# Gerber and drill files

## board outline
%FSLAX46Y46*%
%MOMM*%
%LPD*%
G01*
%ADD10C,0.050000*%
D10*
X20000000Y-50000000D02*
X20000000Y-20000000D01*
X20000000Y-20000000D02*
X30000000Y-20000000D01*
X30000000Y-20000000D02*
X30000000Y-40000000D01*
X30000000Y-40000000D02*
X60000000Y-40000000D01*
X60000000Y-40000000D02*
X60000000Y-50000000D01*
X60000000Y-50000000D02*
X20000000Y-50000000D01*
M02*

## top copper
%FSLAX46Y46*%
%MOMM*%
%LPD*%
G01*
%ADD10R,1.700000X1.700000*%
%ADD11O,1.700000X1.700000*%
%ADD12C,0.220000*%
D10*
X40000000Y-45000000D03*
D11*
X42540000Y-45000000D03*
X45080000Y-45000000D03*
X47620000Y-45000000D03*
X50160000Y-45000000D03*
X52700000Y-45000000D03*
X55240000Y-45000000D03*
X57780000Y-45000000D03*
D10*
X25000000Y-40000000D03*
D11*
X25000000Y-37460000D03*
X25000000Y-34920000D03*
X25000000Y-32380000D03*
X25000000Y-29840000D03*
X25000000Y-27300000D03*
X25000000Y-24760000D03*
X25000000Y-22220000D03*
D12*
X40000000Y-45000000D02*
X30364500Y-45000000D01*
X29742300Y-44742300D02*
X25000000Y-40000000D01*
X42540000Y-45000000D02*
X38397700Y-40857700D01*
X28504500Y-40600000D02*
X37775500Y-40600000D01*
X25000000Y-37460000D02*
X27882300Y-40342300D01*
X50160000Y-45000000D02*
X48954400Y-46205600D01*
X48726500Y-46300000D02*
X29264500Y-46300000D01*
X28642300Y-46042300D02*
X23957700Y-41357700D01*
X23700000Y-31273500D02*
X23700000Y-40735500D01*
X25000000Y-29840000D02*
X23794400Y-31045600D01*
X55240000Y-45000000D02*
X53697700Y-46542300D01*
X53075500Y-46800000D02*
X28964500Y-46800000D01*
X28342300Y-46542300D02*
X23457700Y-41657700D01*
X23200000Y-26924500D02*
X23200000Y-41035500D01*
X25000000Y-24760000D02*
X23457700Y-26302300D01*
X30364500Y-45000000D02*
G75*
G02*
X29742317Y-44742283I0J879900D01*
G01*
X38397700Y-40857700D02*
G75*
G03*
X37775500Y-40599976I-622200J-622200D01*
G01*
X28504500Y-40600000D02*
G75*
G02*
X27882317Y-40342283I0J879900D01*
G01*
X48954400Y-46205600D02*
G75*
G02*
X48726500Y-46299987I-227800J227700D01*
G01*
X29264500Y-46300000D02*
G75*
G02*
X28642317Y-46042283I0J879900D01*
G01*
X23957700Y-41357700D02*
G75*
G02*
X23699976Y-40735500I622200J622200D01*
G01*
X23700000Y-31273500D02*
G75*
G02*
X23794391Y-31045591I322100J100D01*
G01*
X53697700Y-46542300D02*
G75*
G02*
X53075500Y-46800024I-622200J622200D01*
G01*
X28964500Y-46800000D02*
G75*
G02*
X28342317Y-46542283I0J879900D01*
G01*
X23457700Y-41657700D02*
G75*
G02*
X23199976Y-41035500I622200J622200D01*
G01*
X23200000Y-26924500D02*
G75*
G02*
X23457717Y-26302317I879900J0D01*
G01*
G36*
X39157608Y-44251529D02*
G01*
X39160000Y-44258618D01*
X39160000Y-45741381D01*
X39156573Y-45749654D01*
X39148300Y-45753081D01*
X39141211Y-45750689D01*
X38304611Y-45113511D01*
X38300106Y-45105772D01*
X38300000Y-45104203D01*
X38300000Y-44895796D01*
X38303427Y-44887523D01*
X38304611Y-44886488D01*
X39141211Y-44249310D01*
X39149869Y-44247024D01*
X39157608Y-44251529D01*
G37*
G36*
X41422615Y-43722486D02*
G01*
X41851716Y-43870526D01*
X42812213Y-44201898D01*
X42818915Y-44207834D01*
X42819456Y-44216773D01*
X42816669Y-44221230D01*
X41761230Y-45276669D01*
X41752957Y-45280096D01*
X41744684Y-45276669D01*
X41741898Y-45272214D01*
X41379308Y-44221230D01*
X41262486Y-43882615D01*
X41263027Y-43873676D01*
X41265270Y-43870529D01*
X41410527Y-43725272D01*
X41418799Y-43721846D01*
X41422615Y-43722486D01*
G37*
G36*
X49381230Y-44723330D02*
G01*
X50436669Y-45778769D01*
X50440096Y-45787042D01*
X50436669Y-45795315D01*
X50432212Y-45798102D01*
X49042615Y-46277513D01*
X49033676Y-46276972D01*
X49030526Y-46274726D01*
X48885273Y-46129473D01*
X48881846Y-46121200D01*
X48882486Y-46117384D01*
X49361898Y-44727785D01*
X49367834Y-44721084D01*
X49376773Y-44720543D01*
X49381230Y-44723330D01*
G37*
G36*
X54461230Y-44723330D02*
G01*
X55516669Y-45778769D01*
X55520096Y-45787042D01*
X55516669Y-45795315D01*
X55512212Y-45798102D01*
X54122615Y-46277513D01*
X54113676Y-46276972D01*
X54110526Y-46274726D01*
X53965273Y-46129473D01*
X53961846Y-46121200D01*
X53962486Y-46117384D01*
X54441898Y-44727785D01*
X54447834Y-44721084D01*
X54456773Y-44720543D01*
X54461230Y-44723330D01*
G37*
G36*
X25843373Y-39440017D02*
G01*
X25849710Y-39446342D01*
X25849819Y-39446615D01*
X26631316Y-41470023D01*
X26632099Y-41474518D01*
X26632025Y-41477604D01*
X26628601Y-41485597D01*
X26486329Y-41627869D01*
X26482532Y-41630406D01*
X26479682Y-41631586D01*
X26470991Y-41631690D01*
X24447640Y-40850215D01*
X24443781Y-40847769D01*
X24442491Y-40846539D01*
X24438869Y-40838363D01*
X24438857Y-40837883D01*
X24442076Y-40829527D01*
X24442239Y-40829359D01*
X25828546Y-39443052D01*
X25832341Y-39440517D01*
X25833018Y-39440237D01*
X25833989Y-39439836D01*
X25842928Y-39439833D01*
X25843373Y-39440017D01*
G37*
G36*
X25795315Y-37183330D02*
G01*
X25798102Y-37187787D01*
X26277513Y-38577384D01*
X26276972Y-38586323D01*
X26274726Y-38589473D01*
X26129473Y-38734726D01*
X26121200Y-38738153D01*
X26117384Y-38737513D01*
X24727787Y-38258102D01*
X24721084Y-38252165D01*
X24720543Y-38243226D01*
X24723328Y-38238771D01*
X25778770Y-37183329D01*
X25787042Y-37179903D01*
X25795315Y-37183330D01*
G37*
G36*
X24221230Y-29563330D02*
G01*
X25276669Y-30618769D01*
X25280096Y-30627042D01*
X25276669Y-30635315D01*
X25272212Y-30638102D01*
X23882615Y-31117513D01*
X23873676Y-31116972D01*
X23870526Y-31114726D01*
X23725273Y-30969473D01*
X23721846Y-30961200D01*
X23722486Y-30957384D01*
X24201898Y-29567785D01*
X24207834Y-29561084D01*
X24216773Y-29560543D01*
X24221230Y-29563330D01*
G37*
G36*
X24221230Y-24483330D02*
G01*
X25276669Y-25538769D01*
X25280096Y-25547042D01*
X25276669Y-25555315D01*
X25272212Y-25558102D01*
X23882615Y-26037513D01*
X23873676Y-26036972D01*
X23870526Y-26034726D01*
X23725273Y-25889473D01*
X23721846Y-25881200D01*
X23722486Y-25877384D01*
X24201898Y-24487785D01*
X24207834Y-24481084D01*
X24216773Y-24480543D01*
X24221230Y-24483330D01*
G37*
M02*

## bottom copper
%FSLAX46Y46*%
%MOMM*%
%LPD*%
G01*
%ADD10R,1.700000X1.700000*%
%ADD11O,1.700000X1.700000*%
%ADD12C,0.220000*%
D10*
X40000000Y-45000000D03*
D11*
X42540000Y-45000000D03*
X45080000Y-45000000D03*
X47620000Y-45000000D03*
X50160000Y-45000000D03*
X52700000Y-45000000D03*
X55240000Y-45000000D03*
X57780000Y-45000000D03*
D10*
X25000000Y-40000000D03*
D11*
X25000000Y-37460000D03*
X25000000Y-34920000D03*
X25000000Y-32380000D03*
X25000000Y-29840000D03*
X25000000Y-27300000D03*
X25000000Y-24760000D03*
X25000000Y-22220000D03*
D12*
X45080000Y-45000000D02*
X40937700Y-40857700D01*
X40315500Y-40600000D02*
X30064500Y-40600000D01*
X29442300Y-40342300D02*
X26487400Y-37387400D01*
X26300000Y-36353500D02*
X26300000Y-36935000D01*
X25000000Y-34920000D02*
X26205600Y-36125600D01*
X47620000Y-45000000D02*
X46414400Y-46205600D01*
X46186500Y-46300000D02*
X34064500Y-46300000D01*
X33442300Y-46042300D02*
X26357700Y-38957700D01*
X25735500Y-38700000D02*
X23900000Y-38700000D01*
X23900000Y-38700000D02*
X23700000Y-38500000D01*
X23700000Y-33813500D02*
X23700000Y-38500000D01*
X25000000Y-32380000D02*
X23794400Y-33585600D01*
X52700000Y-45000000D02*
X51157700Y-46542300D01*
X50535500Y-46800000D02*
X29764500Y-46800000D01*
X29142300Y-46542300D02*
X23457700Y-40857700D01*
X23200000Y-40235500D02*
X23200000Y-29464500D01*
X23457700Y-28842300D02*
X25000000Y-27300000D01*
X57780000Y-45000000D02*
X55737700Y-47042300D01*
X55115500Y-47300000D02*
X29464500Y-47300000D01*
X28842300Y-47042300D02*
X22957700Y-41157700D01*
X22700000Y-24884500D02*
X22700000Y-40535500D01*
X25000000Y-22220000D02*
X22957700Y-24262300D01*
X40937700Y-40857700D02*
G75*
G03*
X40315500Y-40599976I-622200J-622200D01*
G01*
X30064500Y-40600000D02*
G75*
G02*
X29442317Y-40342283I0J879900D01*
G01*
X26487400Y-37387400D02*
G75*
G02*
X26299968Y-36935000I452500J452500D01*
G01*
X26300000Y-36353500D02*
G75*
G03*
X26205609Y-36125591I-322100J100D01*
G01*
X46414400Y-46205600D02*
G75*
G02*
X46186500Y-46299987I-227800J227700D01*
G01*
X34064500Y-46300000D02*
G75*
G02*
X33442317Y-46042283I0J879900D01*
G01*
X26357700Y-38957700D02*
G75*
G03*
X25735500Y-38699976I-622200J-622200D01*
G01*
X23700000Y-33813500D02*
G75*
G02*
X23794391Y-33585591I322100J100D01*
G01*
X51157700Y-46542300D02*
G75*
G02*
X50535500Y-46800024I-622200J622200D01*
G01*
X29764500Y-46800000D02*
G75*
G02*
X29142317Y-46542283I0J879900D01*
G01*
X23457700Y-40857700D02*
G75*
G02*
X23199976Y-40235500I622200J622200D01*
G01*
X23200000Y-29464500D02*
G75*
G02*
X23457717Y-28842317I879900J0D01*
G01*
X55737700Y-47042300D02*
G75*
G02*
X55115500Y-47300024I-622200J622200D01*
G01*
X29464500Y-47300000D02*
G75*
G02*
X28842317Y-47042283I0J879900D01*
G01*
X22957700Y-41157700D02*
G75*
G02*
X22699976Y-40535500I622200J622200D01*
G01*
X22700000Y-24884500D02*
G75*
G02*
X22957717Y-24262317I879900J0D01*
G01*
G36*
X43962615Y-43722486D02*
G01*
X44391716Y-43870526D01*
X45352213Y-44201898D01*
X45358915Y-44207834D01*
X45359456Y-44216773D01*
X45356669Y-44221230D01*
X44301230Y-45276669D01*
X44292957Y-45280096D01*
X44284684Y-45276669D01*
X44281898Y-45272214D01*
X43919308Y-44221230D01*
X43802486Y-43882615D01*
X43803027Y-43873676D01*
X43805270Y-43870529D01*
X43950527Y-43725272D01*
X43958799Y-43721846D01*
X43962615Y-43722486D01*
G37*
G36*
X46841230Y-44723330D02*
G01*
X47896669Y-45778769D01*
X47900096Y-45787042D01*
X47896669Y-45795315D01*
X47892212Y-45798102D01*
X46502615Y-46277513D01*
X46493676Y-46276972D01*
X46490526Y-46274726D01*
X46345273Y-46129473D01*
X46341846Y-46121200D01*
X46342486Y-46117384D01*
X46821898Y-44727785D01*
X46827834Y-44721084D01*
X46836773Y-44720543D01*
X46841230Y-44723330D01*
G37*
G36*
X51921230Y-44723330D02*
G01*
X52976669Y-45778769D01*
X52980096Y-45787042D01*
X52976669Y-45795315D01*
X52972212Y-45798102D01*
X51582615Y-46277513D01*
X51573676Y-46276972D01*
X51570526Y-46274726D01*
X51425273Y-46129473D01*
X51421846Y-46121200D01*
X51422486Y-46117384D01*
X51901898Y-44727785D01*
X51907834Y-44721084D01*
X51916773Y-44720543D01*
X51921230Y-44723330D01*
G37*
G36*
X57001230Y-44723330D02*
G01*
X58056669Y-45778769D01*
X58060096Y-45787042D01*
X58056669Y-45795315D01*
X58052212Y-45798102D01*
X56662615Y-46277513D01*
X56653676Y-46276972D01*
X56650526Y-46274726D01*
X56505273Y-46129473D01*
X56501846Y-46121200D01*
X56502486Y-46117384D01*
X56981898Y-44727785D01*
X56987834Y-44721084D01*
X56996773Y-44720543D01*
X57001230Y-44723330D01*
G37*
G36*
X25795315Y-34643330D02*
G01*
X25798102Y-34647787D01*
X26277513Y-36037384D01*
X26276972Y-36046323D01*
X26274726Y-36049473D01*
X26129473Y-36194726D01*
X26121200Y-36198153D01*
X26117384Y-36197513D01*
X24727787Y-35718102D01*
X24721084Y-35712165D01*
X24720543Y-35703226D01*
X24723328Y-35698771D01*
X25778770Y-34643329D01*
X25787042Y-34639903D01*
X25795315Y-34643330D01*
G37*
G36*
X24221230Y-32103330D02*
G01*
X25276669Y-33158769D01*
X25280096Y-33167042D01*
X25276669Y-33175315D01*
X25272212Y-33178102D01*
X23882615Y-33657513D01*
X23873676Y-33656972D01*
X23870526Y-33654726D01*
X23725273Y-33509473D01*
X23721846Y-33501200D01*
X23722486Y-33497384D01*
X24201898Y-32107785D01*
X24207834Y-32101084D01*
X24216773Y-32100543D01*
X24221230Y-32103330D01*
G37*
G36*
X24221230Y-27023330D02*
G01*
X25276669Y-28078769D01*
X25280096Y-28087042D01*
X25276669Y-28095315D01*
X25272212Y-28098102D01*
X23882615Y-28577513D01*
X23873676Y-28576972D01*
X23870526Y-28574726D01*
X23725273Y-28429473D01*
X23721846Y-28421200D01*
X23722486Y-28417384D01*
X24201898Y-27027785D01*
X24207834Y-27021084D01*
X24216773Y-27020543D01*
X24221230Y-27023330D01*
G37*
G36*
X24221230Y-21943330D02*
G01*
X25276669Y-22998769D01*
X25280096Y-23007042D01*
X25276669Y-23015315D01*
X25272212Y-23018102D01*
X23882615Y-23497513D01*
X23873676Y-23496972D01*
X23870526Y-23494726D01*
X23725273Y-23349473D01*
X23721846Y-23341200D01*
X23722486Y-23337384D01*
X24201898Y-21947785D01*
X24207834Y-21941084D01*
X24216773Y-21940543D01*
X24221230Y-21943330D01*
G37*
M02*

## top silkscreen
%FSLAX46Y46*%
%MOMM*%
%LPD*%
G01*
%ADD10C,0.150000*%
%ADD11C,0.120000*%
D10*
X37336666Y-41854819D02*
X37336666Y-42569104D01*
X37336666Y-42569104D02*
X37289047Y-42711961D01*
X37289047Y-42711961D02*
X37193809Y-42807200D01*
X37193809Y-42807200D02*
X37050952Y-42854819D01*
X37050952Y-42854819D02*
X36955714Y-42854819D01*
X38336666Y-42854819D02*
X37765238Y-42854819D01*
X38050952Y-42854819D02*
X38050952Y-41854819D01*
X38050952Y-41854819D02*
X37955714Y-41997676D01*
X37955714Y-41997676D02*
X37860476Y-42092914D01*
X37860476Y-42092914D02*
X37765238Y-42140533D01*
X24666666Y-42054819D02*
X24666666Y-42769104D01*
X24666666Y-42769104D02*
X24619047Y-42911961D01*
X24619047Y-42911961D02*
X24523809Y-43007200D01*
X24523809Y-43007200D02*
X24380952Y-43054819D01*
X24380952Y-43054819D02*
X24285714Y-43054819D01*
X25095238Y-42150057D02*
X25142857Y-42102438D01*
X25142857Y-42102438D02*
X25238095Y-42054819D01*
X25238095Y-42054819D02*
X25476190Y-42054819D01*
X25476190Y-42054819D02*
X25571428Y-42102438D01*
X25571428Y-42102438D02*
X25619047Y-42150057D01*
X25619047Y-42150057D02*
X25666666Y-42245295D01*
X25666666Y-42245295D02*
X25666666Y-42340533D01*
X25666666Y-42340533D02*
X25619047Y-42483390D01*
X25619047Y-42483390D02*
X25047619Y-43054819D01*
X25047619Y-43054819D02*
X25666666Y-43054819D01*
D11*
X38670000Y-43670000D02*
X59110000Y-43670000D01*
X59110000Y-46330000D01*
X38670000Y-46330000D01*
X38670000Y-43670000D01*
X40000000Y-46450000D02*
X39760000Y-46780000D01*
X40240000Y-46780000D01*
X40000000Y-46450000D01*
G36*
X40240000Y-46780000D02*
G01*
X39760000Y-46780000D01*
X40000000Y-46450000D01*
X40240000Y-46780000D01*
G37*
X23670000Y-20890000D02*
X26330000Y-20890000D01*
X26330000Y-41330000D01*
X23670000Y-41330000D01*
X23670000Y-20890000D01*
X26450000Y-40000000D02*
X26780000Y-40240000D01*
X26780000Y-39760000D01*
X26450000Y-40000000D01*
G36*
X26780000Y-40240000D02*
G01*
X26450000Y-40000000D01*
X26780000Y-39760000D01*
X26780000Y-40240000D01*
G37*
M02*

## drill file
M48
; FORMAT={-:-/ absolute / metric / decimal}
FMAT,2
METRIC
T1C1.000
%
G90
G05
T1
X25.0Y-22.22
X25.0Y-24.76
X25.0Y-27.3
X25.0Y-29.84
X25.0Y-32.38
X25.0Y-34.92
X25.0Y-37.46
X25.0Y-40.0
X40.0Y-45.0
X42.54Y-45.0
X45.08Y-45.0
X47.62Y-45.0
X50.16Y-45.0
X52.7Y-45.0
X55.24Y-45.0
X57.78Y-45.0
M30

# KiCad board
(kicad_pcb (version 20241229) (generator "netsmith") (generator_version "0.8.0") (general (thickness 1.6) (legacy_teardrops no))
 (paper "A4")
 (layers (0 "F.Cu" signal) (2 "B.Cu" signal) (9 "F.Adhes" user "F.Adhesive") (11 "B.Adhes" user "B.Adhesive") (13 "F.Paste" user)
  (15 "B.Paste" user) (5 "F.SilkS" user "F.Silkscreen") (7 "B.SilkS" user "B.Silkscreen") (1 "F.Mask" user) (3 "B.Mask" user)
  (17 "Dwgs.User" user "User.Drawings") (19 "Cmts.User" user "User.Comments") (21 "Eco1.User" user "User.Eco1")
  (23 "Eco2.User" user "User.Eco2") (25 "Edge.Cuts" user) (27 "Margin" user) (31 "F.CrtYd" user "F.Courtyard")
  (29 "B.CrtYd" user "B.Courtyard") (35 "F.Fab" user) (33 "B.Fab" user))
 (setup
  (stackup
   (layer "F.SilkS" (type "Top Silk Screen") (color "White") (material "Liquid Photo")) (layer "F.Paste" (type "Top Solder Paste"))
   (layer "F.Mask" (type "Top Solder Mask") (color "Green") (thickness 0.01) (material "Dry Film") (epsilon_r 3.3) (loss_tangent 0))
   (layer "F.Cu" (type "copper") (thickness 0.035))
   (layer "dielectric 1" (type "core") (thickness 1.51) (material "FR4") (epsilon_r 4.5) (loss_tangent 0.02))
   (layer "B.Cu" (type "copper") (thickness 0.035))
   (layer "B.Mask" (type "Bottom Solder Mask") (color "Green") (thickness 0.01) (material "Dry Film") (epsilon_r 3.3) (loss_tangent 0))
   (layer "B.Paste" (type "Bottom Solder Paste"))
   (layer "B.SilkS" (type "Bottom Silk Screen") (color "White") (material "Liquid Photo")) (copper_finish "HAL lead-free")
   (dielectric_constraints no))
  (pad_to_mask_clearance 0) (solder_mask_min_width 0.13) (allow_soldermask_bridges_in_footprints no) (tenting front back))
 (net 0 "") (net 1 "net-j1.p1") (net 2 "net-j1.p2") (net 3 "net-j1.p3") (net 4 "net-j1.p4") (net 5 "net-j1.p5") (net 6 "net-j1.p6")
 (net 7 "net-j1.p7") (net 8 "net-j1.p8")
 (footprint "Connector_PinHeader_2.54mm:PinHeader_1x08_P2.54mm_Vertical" (layer "F.Cu") (at 40 45 90)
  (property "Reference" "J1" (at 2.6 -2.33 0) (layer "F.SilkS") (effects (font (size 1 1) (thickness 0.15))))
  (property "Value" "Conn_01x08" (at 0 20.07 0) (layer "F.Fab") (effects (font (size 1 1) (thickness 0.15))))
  (pad "1" thru_hole rect (at 0 0 90) (size 1.7 1.7) (drill 1) (layers "*.Cu" "*.Mask") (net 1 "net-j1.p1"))
  (pad "2" thru_hole oval (at 0 2.54 90) (size 1.7 1.7) (drill 1) (layers "*.Cu" "*.Mask") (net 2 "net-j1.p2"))
  (pad "3" thru_hole oval (at 0 5.08 90) (size 1.7 1.7) (drill 1) (layers "*.Cu" "*.Mask") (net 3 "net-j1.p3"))
  (pad "4" thru_hole oval (at 0 7.62 90) (size 1.7 1.7) (drill 1) (layers "*.Cu" "*.Mask") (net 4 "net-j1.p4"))
  (pad "5" thru_hole oval (at 0 10.16 90) (size 1.7 1.7) (drill 1) (layers "*.Cu" "*.Mask") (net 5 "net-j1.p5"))
  (pad "6" thru_hole oval (at 0 12.7 90) (size 1.7 1.7) (drill 1) (layers "*.Cu" "*.Mask") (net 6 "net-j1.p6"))
  (pad "7" thru_hole oval (at 0 15.24 90) (size 1.7 1.7) (drill 1) (layers "*.Cu" "*.Mask") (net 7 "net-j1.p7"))
  (pad "8" thru_hole oval (at 0 17.78 90) (size 1.7 1.7) (drill 1) (layers "*.Cu" "*.Mask") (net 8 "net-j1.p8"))
  (fp_rect (start -1.33 -1.33) (end 1.33 19.11) (stroke (width 0.12) (type solid)) (fill no) (layer "F.SilkS"))
  (fp_poly (pts (xy -1.45 0) (xy -1.78 -0.24) (xy -1.78 0.24)) (stroke (width 0.12) (type solid)) (fill solid) (layer "F.SilkS")))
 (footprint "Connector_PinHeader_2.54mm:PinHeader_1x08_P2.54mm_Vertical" (layer "F.Cu") (at 25 40 180)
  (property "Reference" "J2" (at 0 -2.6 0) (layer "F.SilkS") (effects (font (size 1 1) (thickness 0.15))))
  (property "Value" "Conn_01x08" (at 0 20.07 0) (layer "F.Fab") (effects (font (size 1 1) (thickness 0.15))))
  (pad "1" thru_hole rect (at 0 0 180) (size 1.7 1.7) (drill 1) (layers "*.Cu" "*.Mask") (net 1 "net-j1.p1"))
  (pad "2" thru_hole oval (at 0 2.54 180) (size 1.7 1.7) (drill 1) (layers "*.Cu" "*.Mask") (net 2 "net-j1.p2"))
  (pad "3" thru_hole oval (at 0 5.08 180) (size 1.7 1.7) (drill 1) (layers "*.Cu" "*.Mask") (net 3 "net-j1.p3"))
  (pad "4" thru_hole oval (at 0 7.62 180) (size 1.7 1.7) (drill 1) (layers "*.Cu" "*.Mask") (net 4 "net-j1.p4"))
  (pad "5" thru_hole oval (at 0 10.16 180) (size 1.7 1.7) (drill 1) (layers "*.Cu" "*.Mask") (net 5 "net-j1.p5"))
  (pad "6" thru_hole oval (at 0 12.7 180) (size 1.7 1.7) (drill 1) (layers "*.Cu" "*.Mask") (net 6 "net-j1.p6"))
  (pad "7" thru_hole oval (at 0 15.24 180) (size 1.7 1.7) (drill 1) (layers "*.Cu" "*.Mask") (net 7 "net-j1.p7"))
  (pad "8" thru_hole oval (at 0 17.78 180) (size 1.7 1.7) (drill 1) (layers "*.Cu" "*.Mask") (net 8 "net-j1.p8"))
  (fp_rect (start -1.33 -1.33) (end 1.33 19.11) (stroke (width 0.12) (type solid)) (fill no) (layer "F.SilkS"))
  (fp_poly (pts (xy -1.45 0) (xy -1.78 -0.24) (xy -1.78 0.24)) (stroke (width 0.12) (type solid)) (fill solid) (layer "F.SilkS")))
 (segment (start 40 45) (end 30.3645 45) (width 0.22) (layer "F.Cu") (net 1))
 (segment (start 29.7423 44.7423) (end 25 40) (width 0.22) (layer "F.Cu") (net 1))
 (segment (start 42.54 45) (end 38.3977 40.8577) (width 0.22) (layer "F.Cu") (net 2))
 (segment (start 28.5045 40.6) (end 37.7755 40.6) (width 0.22) (layer "F.Cu") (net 2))
 (segment (start 25 37.46) (end 27.8823 40.3423) (width 0.22) (layer "F.Cu") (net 2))
 (segment (start 45.08 45) (end 40.9377 40.8577) (width 0.22) (layer "B.Cu") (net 3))
 (segment (start 40.3155 40.6) (end 30.0645 40.6) (width 0.22) (layer "B.Cu") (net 3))
 (segment (start 29.4423 40.3423) (end 26.4874 37.3874) (width 0.22) (layer "B.Cu") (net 3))
 (segment (start 26.3 36.3535) (end 26.3 36.935) (width 0.22) (layer "B.Cu") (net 3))
 (segment (start 25 34.92) (end 26.2056 36.1256) (width 0.22) (layer "B.Cu") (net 3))
 (segment (start 47.62 45) (end 46.4144 46.2056) (width 0.22) (layer "B.Cu") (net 4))
 (segment (start 46.1865 46.3) (end 34.0645 46.3) (width 0.22) (layer "B.Cu") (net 4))
 (segment (start 33.4423 46.0423) (end 26.3577 38.9577) (width 0.22) (layer "B.Cu") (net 4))
 (segment (start 25.7355 38.7) (end 23.9 38.7) (width 0.22) (layer "B.Cu") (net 4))
 (segment (start 23.9 38.7) (end 23.7 38.5) (width 0.22) (layer "B.Cu") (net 4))
 (segment (start 23.7 33.8135) (end 23.7 38.5) (width 0.22) (layer "B.Cu") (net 4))
 (segment (start 25 32.38) (end 23.7944 33.5856) (width 0.22) (layer "B.Cu") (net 4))
 (segment (start 50.16 45) (end 48.9544 46.2056) (width 0.22) (layer "F.Cu") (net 5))
 (segment (start 48.7265 46.3) (end 29.2645 46.3) (width 0.22) (layer "F.Cu") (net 5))
 (segment (start 28.6423 46.0423) (end 23.9577 41.3577) (width 0.22) (layer "F.Cu") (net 5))
 (segment (start 23.7 31.2735) (end 23.7 40.7355) (width 0.22) (layer "F.Cu") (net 5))
 (segment (start 25 29.84) (end 23.7944 31.0456) (width 0.22) (layer "F.Cu") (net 5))
 (segment (start 52.7 45) (end 51.1577 46.5423) (width 0.22) (layer "B.Cu") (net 6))
 (segment (start 50.5355 46.8) (end 29.7645 46.8) (width 0.22) (layer "B.Cu") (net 6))
 (segment (start 29.1423 46.5423) (end 23.4577 40.8577) (width 0.22) (layer "B.Cu") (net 6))
 (segment (start 23.2 40.2355) (end 23.2 29.4645) (width 0.22) (layer "B.Cu") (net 6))
 (segment (start 23.4577 28.8423) (end 25 27.3) (width 0.22) (layer "B.Cu") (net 6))
 (segment (start 55.24 45) (end 53.6977 46.5423) (width 0.22) (layer "F.Cu") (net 7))
 (segment (start 53.0755 46.8) (end 28.9645 46.8) (width 0.22) (layer "F.Cu") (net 7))
 (segment (start 28.3423 46.5423) (end 23.4577 41.6577) (width 0.22) (layer "F.Cu") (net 7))
 (segment (start 23.2 26.9245) (end 23.2 41.0355) (width 0.22) (layer "F.Cu") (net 7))
 (segment (start 25 24.76) (end 23.4577 26.3023) (width 0.22) (layer "F.Cu") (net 7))
 (segment (start 57.78 45) (end 55.7377 47.0423) (width 0.22) (layer "B.Cu") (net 8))
 (segment (start 55.1155 47.3) (end 29.4645 47.3) (width 0.22) (layer "B.Cu") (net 8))
 (segment (start 28.8423 47.0423) (end 22.9577 41.1577) (width 0.22) (layer "B.Cu") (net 8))
 (segment (start 22.7 24.8845) (end 22.7 40.5355) (width 0.22) (layer "B.Cu") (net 8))
 (segment (start 25 22.22) (end 22.9577 24.2623) (width 0.22) (layer "B.Cu") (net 8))
 (arc (start 30.3645 45) (mid 30.0277 44.933) (end 29.7423 44.7423) (width 0.22) (layer "F.Cu") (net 1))
 (arc (start 38.3977 40.8577) (mid 38.1123 40.667) (end 37.7755 40.6) (width 0.22) (layer "F.Cu") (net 2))
 (arc (start 28.5045 40.6) (mid 28.1677 40.533) (end 27.8823 40.3423) (width 0.22) (layer "F.Cu") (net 2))
 (arc (start 40.9377 40.8577) (mid 40.6523 40.667) (end 40.3155 40.6) (width 0.22) (layer "B.Cu") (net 3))
 (arc (start 30.0645 40.6) (mid 29.7277 40.533) (end 29.4423 40.3423) (width 0.22) (layer "B.Cu") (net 3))
 (arc (start 26.4874 37.3874) (mid 26.3487 37.1798) (end 26.3 36.935) (width 0.22) (layer "B.Cu") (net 3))
 (arc (start 26.3 36.3535) (mid 26.2755 36.2302) (end 26.2056 36.1256) (width 0.22) (layer "B.Cu") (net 3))
 (arc (start 46.4144 46.2056) (mid 46.3098 46.2755) (end 46.1865 46.3) (width 0.22) (layer "B.Cu") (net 4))
 (arc (start 34.0645 46.3) (mid 33.7277 46.233) (end 33.4423 46.0423) (width 0.22) (layer "B.Cu") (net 4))
 (arc (start 26.3577 38.9577) (mid 26.0723 38.767) (end 25.7355 38.7) (width 0.22) (layer "B.Cu") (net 4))
 (arc (start 23.7 33.8135) (mid 23.7245 33.6902) (end 23.7944 33.5856) (width 0.22) (layer "B.Cu") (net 4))
 (arc (start 48.9544 46.2056) (mid 48.8498 46.2755) (end 48.7265 46.3) (width 0.22) (layer "F.Cu") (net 5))
 (arc (start 29.2645 46.3) (mid 28.9277 46.233) (end 28.6423 46.0423) (width 0.22) (layer "F.Cu") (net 5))
 (arc (start 23.9577 41.3577) (mid 23.767 41.0723) (end 23.7 40.7355) (width 0.22) (layer "F.Cu") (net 5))
 (arc (start 23.7 31.2735) (mid 23.7245 31.1502) (end 23.7944 31.0456) (width 0.22) (layer "F.Cu") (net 5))
 (arc (start 51.1577 46.5423) (mid 50.8723 46.733) (end 50.5355 46.8) (width 0.22) (layer "B.Cu") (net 6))
 (arc (start 29.7645 46.8) (mid 29.4277 46.733) (end 29.1423 46.5423) (width 0.22) (layer "B.Cu") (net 6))
 (arc (start 23.4577 40.8577) (mid 23.267 40.5723) (end 23.2 40.2355) (width 0.22) (layer "B.Cu") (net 6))
 (arc (start 23.2 29.4645) (mid 23.267 29.1277) (end 23.4577 28.8423) (width 0.22) (layer "B.Cu") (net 6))
 (arc (start 53.6977 46.5423) (mid 53.4123 46.733) (end 53.0755 46.8) (width 0.22) (layer "F.Cu") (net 7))
 (arc (start 28.9645 46.8) (mid 28.6277 46.733) (end 28.3423 46.5423) (width 0.22) (layer "F.Cu") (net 7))
 (arc (start 23.4577 41.6577) (mid 23.267 41.3723) (end 23.2 41.0355) (width 0.22) (layer "F.Cu") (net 7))
 (arc (start 23.2 26.9245) (mid 23.267 26.5877) (end 23.4577 26.3023) (width 0.22) (layer "F.Cu") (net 7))
 (arc (start 55.7377 47.0423) (mid 55.4523 47.233) (end 55.1155 47.3) (width 0.22) (layer "B.Cu") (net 8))
 (arc (start 29.4645 47.3) (mid 29.1277 47.233) (end 28.8423 47.0423) (width 0.22) (layer "B.Cu") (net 8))
 (arc (start 22.9577 41.1577) (mid 22.767 40.8723) (end 22.7 40.5355) (width 0.22) (layer "B.Cu") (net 8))
 (arc (start 22.7 24.8845) (mid 22.767 24.5477) (end 22.9577 24.2623) (width 0.22) (layer "B.Cu") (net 8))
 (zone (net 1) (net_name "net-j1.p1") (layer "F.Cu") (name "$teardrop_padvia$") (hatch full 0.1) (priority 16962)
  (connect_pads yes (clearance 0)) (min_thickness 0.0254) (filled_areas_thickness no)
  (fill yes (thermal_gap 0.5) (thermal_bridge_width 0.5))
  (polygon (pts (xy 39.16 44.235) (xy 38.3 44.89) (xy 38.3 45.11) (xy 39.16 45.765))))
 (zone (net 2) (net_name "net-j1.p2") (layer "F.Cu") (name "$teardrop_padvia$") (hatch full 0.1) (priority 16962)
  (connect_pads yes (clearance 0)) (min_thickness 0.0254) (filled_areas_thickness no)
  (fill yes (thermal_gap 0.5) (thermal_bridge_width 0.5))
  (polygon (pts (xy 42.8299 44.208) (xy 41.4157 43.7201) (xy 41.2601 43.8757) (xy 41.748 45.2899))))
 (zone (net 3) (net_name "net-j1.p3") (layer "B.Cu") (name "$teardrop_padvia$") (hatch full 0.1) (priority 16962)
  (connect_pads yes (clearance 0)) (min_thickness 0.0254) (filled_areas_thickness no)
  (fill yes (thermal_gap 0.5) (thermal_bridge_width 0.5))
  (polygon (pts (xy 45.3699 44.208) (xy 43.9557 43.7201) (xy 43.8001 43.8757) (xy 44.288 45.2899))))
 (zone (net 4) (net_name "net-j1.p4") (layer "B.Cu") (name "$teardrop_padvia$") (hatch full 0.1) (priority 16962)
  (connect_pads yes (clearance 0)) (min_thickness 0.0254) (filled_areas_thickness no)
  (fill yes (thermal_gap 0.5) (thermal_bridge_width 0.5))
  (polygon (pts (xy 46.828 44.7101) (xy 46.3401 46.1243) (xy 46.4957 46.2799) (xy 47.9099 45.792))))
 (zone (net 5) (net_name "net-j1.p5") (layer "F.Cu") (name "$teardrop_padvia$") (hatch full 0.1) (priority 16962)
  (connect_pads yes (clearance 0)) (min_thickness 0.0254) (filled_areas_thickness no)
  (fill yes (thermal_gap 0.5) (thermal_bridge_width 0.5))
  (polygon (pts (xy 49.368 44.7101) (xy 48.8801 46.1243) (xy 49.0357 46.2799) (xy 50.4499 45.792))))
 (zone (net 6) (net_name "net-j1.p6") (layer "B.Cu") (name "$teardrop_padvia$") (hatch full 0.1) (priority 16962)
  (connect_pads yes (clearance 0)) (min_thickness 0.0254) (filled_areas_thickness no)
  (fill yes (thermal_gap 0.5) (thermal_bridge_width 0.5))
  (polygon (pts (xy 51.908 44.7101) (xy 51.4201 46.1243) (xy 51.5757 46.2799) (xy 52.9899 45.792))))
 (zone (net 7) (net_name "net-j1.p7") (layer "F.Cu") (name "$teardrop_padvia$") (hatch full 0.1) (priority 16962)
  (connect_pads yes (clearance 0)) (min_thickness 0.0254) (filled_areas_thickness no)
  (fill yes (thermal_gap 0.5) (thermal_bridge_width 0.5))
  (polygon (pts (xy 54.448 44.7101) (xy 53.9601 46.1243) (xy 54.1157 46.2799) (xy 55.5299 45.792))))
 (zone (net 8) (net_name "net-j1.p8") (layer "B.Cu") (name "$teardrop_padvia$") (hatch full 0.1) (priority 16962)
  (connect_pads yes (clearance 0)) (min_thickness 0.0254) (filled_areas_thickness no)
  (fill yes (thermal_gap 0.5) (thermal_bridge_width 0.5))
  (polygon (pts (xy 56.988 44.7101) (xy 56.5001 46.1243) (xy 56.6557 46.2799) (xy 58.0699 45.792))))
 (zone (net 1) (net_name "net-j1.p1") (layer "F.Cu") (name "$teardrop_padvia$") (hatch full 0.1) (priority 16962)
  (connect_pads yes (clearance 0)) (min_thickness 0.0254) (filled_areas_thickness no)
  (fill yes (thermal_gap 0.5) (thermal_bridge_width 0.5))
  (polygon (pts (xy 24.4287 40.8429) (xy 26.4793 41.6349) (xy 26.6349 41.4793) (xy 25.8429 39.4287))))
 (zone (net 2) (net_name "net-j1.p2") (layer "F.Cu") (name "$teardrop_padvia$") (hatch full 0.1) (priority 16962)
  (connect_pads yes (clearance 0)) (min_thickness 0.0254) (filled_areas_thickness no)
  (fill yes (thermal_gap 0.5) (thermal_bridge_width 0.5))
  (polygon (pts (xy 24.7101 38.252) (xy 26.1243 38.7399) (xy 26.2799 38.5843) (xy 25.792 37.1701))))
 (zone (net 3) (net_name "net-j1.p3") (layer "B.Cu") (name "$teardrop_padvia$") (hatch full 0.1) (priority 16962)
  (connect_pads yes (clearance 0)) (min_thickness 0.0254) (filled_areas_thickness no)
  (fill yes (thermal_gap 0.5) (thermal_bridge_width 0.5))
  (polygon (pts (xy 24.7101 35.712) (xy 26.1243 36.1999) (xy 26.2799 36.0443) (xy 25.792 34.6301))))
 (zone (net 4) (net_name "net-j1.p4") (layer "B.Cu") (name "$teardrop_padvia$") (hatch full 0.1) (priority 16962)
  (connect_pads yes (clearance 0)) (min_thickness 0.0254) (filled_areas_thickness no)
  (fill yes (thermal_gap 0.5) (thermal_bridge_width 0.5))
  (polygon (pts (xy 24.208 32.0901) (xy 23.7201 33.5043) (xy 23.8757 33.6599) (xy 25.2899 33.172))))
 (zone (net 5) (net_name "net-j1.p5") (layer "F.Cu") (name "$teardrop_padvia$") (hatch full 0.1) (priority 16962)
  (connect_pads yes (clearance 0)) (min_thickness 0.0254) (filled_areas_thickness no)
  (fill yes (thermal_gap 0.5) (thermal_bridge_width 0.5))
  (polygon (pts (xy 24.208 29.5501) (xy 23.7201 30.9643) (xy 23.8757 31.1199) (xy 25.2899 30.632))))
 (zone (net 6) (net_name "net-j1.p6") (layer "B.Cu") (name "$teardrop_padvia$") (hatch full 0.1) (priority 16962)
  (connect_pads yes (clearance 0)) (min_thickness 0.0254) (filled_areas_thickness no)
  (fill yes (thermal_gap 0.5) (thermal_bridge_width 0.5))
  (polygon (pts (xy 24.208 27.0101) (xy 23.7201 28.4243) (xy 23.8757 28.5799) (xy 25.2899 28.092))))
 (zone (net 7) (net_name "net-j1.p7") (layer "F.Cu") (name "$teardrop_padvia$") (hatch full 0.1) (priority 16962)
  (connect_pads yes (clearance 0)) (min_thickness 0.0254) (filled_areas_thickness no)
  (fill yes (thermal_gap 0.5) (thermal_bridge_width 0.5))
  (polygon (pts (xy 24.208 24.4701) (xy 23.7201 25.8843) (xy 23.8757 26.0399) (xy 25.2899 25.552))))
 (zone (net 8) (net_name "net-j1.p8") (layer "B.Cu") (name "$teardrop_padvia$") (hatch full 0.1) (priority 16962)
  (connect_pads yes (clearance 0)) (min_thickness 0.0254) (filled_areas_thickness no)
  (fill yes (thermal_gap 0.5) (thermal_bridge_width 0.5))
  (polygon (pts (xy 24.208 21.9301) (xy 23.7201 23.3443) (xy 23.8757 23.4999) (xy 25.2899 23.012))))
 (gr_line (start 20 50) (end 20 20) (stroke (width 0.05) (type default)) (layer "Edge.Cuts"))
 (gr_line (start 20 20) (end 30 20) (stroke (width 0.05) (type default)) (layer "Edge.Cuts"))
 (gr_line (start 30 20) (end 30 40) (stroke (width 0.05) (type default)) (layer "Edge.Cuts"))
 (gr_line (start 30 40) (end 60 40) (stroke (width 0.05) (type default)) (layer "Edge.Cuts"))
 (gr_line (start 60 40) (end 60 50) (stroke (width 0.05) (type default)) (layer "Edge.Cuts"))
 (gr_line (start 60 50) (end 20 50) (stroke (width 0.05) (type default)) (layer "Edge.Cuts")))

